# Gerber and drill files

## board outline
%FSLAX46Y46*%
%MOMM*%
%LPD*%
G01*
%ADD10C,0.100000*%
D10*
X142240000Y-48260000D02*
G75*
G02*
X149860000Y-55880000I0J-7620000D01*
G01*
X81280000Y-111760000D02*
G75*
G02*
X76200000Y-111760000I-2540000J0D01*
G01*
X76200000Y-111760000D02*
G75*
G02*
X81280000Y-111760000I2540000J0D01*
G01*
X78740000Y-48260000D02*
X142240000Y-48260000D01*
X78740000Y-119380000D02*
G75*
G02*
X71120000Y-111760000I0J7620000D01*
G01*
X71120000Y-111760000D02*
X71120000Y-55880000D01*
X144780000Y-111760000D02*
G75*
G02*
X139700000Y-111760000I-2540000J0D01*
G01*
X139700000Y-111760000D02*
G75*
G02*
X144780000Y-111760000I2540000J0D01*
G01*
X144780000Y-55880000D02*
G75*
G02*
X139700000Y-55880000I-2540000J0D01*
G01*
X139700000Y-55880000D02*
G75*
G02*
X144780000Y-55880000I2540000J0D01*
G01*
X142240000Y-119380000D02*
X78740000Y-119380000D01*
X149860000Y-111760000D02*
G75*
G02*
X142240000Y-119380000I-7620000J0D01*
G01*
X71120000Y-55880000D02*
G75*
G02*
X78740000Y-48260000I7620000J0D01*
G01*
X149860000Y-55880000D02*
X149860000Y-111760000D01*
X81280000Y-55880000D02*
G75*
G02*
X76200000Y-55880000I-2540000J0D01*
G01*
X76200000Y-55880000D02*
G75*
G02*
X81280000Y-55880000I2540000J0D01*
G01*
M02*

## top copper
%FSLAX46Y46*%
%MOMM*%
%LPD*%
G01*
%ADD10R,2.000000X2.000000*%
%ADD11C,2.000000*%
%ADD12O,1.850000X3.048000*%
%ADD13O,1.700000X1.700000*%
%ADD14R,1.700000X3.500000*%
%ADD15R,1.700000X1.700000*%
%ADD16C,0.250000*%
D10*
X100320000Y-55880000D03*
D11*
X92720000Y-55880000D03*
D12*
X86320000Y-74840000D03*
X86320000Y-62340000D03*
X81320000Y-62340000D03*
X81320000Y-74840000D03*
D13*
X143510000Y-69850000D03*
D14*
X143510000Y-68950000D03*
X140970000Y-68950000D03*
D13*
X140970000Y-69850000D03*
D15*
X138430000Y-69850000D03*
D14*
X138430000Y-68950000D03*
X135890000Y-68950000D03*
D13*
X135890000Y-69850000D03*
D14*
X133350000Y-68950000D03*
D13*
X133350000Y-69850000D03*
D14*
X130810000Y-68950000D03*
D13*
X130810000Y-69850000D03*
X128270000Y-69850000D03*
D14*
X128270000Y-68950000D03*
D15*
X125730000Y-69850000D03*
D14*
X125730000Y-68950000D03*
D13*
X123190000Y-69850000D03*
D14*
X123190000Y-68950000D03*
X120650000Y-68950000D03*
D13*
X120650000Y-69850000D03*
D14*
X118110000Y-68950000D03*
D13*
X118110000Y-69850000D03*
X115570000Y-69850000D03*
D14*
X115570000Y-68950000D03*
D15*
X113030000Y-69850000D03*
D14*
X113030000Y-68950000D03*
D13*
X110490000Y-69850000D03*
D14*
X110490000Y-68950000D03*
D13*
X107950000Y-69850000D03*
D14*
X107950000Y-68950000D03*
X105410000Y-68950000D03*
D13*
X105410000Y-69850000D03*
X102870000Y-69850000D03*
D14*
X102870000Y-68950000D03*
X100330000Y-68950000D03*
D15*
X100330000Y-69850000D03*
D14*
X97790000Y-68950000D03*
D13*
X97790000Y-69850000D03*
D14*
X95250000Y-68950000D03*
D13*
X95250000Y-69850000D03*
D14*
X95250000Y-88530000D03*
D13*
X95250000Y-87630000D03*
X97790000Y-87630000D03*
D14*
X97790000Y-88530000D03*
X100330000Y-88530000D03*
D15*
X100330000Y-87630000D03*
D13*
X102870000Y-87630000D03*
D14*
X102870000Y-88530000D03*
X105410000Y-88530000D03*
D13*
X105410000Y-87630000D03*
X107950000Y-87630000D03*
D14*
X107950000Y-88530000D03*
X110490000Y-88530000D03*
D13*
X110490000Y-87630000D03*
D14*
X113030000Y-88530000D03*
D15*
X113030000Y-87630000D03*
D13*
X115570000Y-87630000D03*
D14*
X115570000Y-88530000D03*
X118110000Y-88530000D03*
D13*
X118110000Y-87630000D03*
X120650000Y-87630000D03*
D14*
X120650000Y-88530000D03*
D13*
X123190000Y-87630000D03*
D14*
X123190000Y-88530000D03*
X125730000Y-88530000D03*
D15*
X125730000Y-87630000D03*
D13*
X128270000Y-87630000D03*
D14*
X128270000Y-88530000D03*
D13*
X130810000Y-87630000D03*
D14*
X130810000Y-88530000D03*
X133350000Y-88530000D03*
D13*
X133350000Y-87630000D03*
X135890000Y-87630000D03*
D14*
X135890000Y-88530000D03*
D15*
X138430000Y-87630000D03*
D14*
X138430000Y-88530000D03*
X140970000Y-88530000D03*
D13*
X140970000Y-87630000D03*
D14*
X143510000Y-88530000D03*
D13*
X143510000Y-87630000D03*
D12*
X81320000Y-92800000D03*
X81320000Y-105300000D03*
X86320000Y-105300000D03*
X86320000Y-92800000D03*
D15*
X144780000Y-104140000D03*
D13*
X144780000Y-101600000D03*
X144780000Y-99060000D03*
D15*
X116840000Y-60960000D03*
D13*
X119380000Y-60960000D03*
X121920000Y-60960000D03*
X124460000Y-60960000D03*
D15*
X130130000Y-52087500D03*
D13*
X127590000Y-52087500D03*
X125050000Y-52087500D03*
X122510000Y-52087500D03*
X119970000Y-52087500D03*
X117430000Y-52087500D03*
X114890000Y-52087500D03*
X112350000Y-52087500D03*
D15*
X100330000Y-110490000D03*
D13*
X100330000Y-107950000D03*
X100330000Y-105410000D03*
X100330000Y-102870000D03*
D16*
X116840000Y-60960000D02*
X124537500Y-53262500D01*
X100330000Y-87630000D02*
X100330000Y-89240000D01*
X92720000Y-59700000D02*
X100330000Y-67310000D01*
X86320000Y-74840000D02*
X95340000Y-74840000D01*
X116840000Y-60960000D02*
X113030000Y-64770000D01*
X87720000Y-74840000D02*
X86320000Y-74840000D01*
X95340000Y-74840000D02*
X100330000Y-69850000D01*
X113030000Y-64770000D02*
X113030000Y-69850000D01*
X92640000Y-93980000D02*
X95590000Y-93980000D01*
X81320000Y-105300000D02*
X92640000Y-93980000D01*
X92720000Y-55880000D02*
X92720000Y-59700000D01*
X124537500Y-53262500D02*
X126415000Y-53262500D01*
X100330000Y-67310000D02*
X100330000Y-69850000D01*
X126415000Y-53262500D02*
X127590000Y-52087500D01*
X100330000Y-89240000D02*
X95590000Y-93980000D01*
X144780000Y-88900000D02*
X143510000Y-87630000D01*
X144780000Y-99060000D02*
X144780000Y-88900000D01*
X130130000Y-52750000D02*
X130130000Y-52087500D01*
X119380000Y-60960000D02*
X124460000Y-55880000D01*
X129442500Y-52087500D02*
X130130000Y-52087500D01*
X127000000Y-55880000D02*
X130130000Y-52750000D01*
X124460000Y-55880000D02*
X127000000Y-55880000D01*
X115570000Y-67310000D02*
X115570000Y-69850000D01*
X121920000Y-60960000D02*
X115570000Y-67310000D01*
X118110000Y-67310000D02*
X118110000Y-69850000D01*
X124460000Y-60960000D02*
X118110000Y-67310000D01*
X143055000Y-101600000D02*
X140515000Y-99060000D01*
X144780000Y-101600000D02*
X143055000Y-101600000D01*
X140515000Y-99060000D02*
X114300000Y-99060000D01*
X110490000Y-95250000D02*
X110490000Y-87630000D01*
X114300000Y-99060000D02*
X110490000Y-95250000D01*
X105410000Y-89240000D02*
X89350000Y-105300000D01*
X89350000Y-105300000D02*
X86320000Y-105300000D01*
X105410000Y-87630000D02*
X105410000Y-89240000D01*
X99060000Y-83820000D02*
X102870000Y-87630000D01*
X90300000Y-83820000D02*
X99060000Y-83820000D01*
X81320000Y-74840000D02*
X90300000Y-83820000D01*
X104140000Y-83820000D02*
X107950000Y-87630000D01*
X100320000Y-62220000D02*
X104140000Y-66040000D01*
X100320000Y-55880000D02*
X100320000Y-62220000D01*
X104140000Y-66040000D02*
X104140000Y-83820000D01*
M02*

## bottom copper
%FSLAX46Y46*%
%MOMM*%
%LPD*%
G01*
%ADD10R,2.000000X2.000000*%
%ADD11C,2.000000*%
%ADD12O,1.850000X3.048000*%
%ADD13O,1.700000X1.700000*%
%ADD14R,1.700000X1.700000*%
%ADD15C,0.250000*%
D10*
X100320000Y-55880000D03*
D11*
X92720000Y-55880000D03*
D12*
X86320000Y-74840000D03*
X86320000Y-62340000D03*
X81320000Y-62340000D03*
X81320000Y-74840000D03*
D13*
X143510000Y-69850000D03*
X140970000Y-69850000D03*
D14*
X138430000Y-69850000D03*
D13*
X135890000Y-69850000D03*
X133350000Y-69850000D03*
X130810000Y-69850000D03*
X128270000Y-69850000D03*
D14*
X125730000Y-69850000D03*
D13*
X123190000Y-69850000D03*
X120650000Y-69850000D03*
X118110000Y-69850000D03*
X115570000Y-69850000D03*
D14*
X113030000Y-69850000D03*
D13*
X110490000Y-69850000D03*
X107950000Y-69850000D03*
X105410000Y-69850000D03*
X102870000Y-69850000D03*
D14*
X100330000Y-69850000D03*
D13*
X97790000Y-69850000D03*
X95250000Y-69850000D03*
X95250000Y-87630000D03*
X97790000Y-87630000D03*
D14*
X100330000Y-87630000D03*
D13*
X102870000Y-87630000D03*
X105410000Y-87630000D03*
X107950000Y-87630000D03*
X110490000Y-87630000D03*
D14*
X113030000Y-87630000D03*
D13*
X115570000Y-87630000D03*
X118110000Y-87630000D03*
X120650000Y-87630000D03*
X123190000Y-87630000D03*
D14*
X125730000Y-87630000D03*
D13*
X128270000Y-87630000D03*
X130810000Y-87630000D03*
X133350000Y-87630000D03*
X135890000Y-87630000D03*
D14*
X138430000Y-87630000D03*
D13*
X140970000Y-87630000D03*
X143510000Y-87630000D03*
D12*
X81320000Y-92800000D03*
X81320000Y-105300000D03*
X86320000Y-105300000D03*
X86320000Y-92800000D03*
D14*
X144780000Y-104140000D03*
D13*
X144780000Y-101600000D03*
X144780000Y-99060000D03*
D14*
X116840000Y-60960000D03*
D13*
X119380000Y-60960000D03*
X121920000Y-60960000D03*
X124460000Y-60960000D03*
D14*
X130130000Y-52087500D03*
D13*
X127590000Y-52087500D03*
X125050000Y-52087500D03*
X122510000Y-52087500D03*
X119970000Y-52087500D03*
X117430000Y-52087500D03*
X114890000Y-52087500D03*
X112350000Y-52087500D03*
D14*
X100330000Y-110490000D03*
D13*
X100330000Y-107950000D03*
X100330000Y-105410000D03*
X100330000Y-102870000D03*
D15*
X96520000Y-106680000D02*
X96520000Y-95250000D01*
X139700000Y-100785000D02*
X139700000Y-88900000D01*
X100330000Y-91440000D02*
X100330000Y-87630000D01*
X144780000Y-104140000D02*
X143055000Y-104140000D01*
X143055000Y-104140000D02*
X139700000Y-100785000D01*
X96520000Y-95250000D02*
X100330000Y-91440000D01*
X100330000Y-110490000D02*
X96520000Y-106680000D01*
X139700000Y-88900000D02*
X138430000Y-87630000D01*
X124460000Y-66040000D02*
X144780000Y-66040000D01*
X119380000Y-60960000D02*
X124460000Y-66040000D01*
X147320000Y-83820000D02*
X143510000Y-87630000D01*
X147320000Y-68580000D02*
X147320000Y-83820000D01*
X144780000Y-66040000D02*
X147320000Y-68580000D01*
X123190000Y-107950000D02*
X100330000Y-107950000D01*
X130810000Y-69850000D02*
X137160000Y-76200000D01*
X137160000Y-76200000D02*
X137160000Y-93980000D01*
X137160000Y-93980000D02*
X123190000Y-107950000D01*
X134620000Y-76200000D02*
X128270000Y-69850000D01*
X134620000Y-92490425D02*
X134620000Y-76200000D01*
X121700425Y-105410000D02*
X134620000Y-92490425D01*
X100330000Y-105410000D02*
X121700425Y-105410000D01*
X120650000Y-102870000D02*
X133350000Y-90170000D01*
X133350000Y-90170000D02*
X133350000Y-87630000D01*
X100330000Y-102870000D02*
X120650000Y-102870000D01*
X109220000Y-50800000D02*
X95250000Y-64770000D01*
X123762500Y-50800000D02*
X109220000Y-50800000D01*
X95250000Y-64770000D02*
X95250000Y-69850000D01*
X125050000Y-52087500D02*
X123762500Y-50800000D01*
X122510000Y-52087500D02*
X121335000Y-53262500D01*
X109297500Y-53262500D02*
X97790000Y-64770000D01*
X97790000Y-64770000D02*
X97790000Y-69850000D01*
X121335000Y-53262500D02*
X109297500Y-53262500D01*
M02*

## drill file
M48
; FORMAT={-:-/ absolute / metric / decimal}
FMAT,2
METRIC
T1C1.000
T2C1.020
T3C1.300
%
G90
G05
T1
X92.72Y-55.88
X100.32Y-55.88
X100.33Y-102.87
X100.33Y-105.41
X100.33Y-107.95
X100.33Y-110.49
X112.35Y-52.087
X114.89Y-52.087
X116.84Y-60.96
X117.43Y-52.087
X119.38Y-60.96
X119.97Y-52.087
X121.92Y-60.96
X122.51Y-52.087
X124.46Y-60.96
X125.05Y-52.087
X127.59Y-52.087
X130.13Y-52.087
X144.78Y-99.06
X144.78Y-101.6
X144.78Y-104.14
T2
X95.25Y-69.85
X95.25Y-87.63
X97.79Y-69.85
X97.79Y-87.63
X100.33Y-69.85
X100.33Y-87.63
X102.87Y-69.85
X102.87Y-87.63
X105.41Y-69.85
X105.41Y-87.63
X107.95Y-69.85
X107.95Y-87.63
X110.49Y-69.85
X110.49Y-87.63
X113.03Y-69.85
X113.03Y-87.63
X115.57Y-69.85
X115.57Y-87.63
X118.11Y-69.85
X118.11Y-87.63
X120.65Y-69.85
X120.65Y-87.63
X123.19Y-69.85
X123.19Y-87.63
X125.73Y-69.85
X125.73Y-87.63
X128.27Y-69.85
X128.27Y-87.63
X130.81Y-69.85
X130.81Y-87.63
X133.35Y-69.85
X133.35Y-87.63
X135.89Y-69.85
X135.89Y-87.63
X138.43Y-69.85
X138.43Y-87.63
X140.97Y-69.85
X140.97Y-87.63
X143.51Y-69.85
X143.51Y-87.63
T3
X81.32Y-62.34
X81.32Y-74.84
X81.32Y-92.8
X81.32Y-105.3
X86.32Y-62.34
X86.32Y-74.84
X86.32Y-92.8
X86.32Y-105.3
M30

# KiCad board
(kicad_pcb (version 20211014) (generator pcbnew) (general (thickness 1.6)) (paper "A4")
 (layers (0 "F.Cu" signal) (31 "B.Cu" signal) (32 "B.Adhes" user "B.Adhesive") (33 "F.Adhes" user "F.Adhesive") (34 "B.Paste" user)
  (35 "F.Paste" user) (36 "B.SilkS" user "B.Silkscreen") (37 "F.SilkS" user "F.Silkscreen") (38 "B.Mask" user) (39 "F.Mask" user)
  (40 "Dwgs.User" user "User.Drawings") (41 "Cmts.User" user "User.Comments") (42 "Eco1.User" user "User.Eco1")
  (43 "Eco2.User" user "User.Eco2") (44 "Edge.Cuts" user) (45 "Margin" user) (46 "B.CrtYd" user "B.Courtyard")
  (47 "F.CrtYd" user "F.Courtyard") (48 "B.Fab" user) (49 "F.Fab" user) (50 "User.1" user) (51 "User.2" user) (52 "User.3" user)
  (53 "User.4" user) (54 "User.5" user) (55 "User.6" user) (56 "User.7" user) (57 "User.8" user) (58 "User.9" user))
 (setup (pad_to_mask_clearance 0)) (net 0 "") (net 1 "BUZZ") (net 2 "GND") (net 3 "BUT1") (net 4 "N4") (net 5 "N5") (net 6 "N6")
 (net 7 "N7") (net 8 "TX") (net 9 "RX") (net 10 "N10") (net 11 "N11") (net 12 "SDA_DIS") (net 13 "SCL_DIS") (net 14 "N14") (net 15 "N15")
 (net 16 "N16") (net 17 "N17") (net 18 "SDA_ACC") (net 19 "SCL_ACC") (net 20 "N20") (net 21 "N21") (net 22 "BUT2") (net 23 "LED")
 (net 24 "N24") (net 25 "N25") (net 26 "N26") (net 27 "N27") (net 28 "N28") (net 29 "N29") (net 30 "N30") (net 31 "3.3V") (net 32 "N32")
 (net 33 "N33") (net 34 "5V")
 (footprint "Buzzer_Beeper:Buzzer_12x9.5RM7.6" (layer "F.Cu") (at 100.32 55.88 180)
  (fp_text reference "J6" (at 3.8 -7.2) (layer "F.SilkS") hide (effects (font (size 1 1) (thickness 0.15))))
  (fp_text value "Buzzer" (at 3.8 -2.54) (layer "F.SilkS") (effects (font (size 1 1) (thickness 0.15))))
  (pad "1" thru_hole rect (at 0 0 180) (size 2 2) (drill 1) (layers *.Cu *.Mask) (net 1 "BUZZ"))
  (pad "2" thru_hole circle (at 7.6 0 180) (size 2 2) (drill 1) (layers *.Cu *.Mask) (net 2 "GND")))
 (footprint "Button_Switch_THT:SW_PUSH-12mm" (layer "F.Cu") (at 86.32 62.34 -90)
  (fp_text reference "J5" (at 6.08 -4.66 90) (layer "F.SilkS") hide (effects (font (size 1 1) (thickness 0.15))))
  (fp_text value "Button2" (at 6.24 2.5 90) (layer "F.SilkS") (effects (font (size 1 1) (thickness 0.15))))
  (pad "1" thru_hole oval (at 12.5 0 270) (size 3.048 1.85) (drill 1.3) (layers *.Cu *.Mask) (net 2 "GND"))
  (pad "1" thru_hole oval (at 0 0 270) (size 3.048 1.85) (drill 1.3) (layers *.Cu *.Mask) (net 2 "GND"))
  (pad "2" thru_hole oval (at 0 5 270) (size 3.048 1.85) (drill 1.3) (layers *.Cu *.Mask) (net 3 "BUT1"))
  (pad "2" thru_hole oval (at 12.5 5 270) (size 3.048 1.85) (drill 1.3) (layers *.Cu *.Mask) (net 3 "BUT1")))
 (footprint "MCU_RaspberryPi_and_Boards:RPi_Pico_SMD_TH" (layer "F.Cu") (at 119.38 78.74 -90)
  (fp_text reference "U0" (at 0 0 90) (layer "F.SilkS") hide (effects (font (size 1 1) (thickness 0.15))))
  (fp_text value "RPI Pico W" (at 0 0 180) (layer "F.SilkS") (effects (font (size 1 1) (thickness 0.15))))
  (pad "1" thru_hole oval (at -8.89 -24.13 270) (size 1.7 1.7) (drill 1.02) (layers *.Cu *.Mask) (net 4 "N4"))
  (pad "1" smd rect (at -8.89 -24.13 270) (size 3.5 1.7) (drill (offset -0.9 0)) (layers "F.Cu" "F.Mask") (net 4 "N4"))
  (pad "2" smd rect (at -8.89 -21.59 270) (size 3.5 1.7) (drill (offset -0.9 0)) (layers "F.Cu" "F.Mask") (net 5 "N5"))
  (pad "2" thru_hole oval (at -8.89 -21.59 270) (size 1.7 1.7) (drill 1.02) (layers *.Cu *.Mask) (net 5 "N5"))
  (pad "3" thru_hole rect (at -8.89 -19.05 270) (size 1.7 1.7) (drill 1.02) (layers *.Cu *.Mask) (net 2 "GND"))
  (pad "3" smd rect (at -8.89 -19.05 270) (size 3.5 1.7) (drill (offset -0.9 0)) (layers "F.Cu" "F.Mask") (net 2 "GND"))
  (pad "4" smd rect (at -8.89 -16.51 270) (size 3.5 1.7) (drill (offset -0.9 0)) (layers "F.Cu" "F.Mask") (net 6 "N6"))
  (pad "4" thru_hole oval (at -8.89 -16.51 270) (size 1.7 1.7) (drill 1.02) (layers *.Cu *.Mask) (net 6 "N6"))
  (pad "5" smd rect (at -8.89 -13.97 270) (size 3.5 1.7) (drill (offset -0.9 0)) (layers "F.Cu" "F.Mask") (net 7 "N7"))
  (pad "5" thru_hole oval (at -8.89 -13.97 270) (size 1.7 1.7) (drill 1.02) (layers *.Cu *.Mask) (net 7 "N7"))
  (pad "6" smd rect (at -8.89 -11.43 270) (size 3.5 1.7) (drill (offset -0.9 0)) (layers "F.Cu" "F.Mask") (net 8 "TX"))
  (pad "6" thru_hole oval (at -8.89 -11.43 270) (size 1.7 1.7) (drill 1.02) (layers *.Cu *.Mask) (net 8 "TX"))
  (pad "7" thru_hole oval (at -8.89 -8.89 270) (size 1.7 1.7) (drill 1.02) (layers *.Cu *.Mask) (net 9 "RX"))
  (pad "7" smd rect (at -8.89 -8.89 270) (size 3.5 1.7) (drill (offset -0.9 0)) (layers "F.Cu" "F.Mask") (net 9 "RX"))
  (pad "8" thru_hole rect (at -8.89 -6.35 270) (size 1.7 1.7) (drill 1.02) (layers *.Cu *.Mask) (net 2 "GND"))
  (pad "8" smd rect (at -8.89 -6.35 270) (size 3.5 1.7) (drill (offset -0.9 0)) (layers "F.Cu" "F.Mask") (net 2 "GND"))
  (pad "9" thru_hole oval (at -8.89 -3.81 270) (size 1.7 1.7) (drill 1.02) (layers *.Cu *.Mask) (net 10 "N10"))
  (pad "9" smd rect (at -8.89 -3.81 270) (size 3.5 1.7) (drill (offset -0.9 0)) (layers "F.Cu" "F.Mask") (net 10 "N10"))
  (pad "10" smd rect (at -8.89 -1.27 270) (size 3.5 1.7) (drill (offset -0.9 0)) (layers "F.Cu" "F.Mask") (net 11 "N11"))
  (pad "10" thru_hole oval (at -8.89 -1.27 270) (size 1.7 1.7) (drill 1.02) (layers *.Cu *.Mask) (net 11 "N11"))
  (pad "11" smd rect (at -8.89 1.27 270) (size 3.5 1.7) (drill (offset -0.9 0)) (layers "F.Cu" "F.Mask") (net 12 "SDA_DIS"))
  (pad "11" thru_hole oval (at -8.89 1.27 270) (size 1.7 1.7) (drill 1.02) (layers *.Cu *.Mask) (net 12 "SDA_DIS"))
  (pad "12" thru_hole oval (at -8.89 3.81 270) (size 1.7 1.7) (drill 1.02) (layers *.Cu *.Mask) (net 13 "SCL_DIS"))
  (pad "12" smd rect (at -8.89 3.81 270) (size 3.5 1.7) (drill (offset -0.9 0)) (layers "F.Cu" "F.Mask") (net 13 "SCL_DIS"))
  (pad "13" thru_hole rect (at -8.89 6.35 270) (size 1.7 1.7) (drill 1.02) (layers *.Cu *.Mask) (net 2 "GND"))
  (pad "13" smd rect (at -8.89 6.35 270) (size 3.5 1.7) (drill (offset -0.9 0)) (layers "F.Cu" "F.Mask") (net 2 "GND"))
  (pad "14" thru_hole oval (at -8.89 8.89 270) (size 1.7 1.7) (drill 1.02) (layers *.Cu *.Mask) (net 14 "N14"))
  (pad "14" smd rect (at -8.89 8.89 270) (size 3.5 1.7) (drill (offset -0.9 0)) (layers "F.Cu" "F.Mask") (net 14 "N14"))
  (pad "15" thru_hole oval (at -8.89 11.43 270) (size 1.7 1.7) (drill 1.02) (layers *.Cu *.Mask) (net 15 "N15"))
  (pad "15" smd rect (at -8.89 11.43 270) (size 3.5 1.7) (drill (offset -0.9 0)) (layers "F.Cu" "F.Mask") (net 15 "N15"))
  (pad "16" smd rect (at -8.89 13.97 270) (size 3.5 1.7) (drill (offset -0.9 0)) (layers "F.Cu" "F.Mask") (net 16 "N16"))
  (pad "16" thru_hole oval (at -8.89 13.97 270) (size 1.7 1.7) (drill 1.02) (layers *.Cu *.Mask) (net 16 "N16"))
  (pad "17" thru_hole oval (at -8.89 16.51 270) (size 1.7 1.7) (drill 1.02) (layers *.Cu *.Mask) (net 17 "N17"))
  (pad "17" smd rect (at -8.89 16.51 270) (size 3.5 1.7) (drill (offset -0.9 0)) (layers "F.Cu" "F.Mask") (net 17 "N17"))
  (pad "18" smd rect (at -8.89 19.05 270) (size 3.5 1.7) (drill (offset -0.9 0)) (layers "F.Cu" "F.Mask") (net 2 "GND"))
  (pad "18" thru_hole rect (at -8.89 19.05 270) (size 1.7 1.7) (drill 1.02) (layers *.Cu *.Mask) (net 2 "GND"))
  (pad "19" smd rect (at -8.89 21.59 270) (size 3.5 1.7) (drill (offset -0.9 0)) (layers "F.Cu" "F.Mask") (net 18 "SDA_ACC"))
  (pad "19" thru_hole oval (at -8.89 21.59 270) (size 1.7 1.7) (drill 1.02) (layers *.Cu *.Mask) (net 18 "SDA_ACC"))
  (pad "20" smd rect (at -8.89 24.13 270) (size 3.5 1.7) (drill (offset -0.9 0)) (layers "F.Cu" "F.Mask") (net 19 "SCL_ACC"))
  (pad "20" thru_hole oval (at -8.89 24.13 270) (size 1.7 1.7) (drill 1.02) (layers *.Cu *.Mask) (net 19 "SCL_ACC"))
  (pad "21" smd rect (at 8.89 24.13 270) (size 3.5 1.7) (drill (offset 0.9 0)) (layers "F.Cu" "F.Mask") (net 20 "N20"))
  (pad "21" thru_hole oval (at 8.89 24.13 270) (size 1.7 1.7) (drill 1.02) (layers *.Cu *.Mask) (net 20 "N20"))
  (pad "22" thru_hole oval (at 8.89 21.59 270) (size 1.7 1.7) (drill 1.02) (layers *.Cu *.Mask) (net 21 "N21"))
  (pad "22" smd rect (at 8.89 21.59 270) (size 3.5 1.7) (drill (offset 0.9 0)) (layers "F.Cu" "F.Mask") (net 21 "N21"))
  (pad "23" smd rect (at 8.89 19.05 270) (size 3.5 1.7) (drill (offset 0.9 0)) (layers "F.Cu" "F.Mask") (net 2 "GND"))
  (pad "23" thru_hole rect (at 8.89 19.05 270) (size 1.7 1.7) (drill 1.02) (layers *.Cu *.Mask) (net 2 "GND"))
  (pad "24" thru_hole oval (at 8.89 16.51 270) (size 1.7 1.7) (drill 1.02) (layers *.Cu *.Mask) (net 3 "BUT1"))
  (pad "24" smd rect (at 8.89 16.51 270) (size 3.5 1.7) (drill (offset 0.9 0)) (layers "F.Cu" "F.Mask") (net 3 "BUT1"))
  (pad "25" smd rect (at 8.89 13.97 270) (size 3.5 1.7) (drill (offset 0.9 0)) (layers "F.Cu" "F.Mask") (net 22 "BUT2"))
  (pad "25" thru_hole oval (at 8.89 13.97 270) (size 1.7 1.7) (drill 1.02) (layers *.Cu *.Mask) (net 22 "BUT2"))
  (pad "26" thru_hole oval (at 8.89 11.43 270) (size 1.7 1.7) (drill 1.02) (layers *.Cu *.Mask) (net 1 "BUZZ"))
  (pad "26" smd rect (at 8.89 11.43 270) (size 3.5 1.7) (drill (offset 0.9 0)) (layers "F.Cu" "F.Mask") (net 1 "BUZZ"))
  (pad "27" smd rect (at 8.89 8.89 270) (size 3.5 1.7) (drill (offset 0.9 0)) (layers "F.Cu" "F.Mask") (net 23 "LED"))
  (pad "27" thru_hole oval (at 8.89 8.89 270) (size 1.7 1.7) (drill 1.02) (layers *.Cu *.Mask) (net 23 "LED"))
  (pad "28" smd rect (at 8.89 6.35 270) (size 3.5 1.7) (drill (offset 0.9 0)) (layers "F.Cu" "F.Mask") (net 2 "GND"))
  (pad "28" thru_hole rect (at 8.89 6.35 270) (size 1.7 1.7) (drill 1.02) (layers *.Cu *.Mask) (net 2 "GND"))
  (pad "29" thru_hole oval (at 8.89 3.81 270) (size 1.7 1.7) (drill 1.02) (layers *.Cu *.Mask) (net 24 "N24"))
  (pad "29" smd rect (at 8.89 3.81 270) (size 3.5 1.7) (drill (offset 0.9 0)) (layers "F.Cu" "F.Mask") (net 24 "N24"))
  (pad "30" smd rect (at 8.89 1.27 270) (size 3.5 1.7) (drill (offset 0.9 0)) (layers "F.Cu" "F.Mask") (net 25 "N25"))
  (pad "30" thru_hole oval (at 8.89 1.27 270) (size 1.7 1.7) (drill 1.02) (layers *.Cu *.Mask) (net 25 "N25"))
  (pad "31" thru_hole oval (at 8.89 -1.27 270) (size 1.7 1.7) (drill 1.02) (layers *.Cu *.Mask) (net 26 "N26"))
  (pad "31" smd rect (at 8.89 -1.27 270) (size 3.5 1.7) (drill (offset 0.9 0)) (layers "F.Cu" "F.Mask") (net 26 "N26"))
  (pad "32" thru_hole oval (at 8.89 -3.81 270) (size 1.7 1.7) (drill 1.02) (layers *.Cu *.Mask) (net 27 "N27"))
  (pad "32" smd rect (at 8.89 -3.81 270) (size 3.5 1.7) (drill (offset 0.9 0)) (layers "F.Cu" "F.Mask") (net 27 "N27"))
  (pad "33" smd rect (at 8.89 -6.35 270) (size 3.5 1.7) (drill (offset 0.9 0)) (layers "F.Cu" "F.Mask") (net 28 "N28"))
  (pad "33" thru_hole rect (at 8.89 -6.35 270) (size 1.7 1.7) (drill 1.02) (layers *.Cu *.Mask) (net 28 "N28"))
  (pad "34" thru_hole oval (at 8.89 -8.89 270) (size 1.7 1.7) (drill 1.02) (layers *.Cu *.Mask) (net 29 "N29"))
  (pad "34" smd rect (at 8.89 -8.89 270) (size 3.5 1.7) (drill (offset 0.9 0)) (layers "F.Cu" "F.Mask") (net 29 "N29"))
  (pad "35" thru_hole oval (at 8.89 -11.43 270) (size 1.7 1.7) (drill 1.02) (layers *.Cu *.Mask) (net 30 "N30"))
  (pad "35" smd rect (at 8.89 -11.43 270) (size 3.5 1.7) (drill (offset 0.9 0)) (layers "F.Cu" "F.Mask") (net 30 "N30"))
  (pad "36" smd rect (at 8.89 -13.97 270) (size 3.5 1.7) (drill (offset 0.9 0)) (layers "F.Cu" "F.Mask") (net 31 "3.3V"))
  (pad "36" thru_hole oval (at 8.89 -13.97 270) (size 1.7 1.7) (drill 1.02) (layers *.Cu *.Mask) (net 31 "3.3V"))
  (pad "37" thru_hole oval (at 8.89 -16.51 270) (size 1.7 1.7) (drill 1.02) (layers *.Cu *.Mask) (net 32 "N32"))
  (pad "37" smd rect (at 8.89 -16.51 270) (size 3.5 1.7) (drill (offset 0.9 0)) (layers "F.Cu" "F.Mask") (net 32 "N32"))
  (pad "38" thru_hole rect (at 8.89 -19.05 270) (size 1.7 1.7) (drill 1.02) (layers *.Cu *.Mask) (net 2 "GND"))
  (pad "38" smd rect (at 8.89 -19.05 270) (size 3.5 1.7) (drill (offset 0.9 0)) (layers "F.Cu" "F.Mask") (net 2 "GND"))
  (pad "39" smd rect (at 8.89 -21.59 270) (size 3.5 1.7) (drill (offset 0.9 0)) (layers "F.Cu" "F.Mask") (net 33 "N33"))
  (pad "39" thru_hole oval (at 8.89 -21.59 270) (size 1.7 1.7) (drill 1.02) (layers *.Cu *.Mask) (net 33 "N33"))
  (pad "40" smd rect (at 8.89 -24.13 270) (size 3.5 1.7) (drill (offset 0.9 0)) (layers "F.Cu" "F.Mask") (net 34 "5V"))
  (pad "40" thru_hole oval (at 8.89 -24.13 270) (size 1.7 1.7) (drill 1.02) (layers *.Cu *.Mask) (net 34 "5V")))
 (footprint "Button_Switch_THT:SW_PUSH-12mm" (layer "F.Cu") (at 81.32 105.3 90)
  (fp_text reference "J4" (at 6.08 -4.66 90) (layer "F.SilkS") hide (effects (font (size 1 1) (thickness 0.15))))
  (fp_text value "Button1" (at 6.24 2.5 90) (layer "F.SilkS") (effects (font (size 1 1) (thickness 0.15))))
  (pad "1" thru_hole oval (at 12.5 0 90) (size 3.048 1.85) (drill 1.3) (layers *.Cu *.Mask) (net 2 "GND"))
  (pad "1" thru_hole oval (at 0 0 90) (size 3.048 1.85) (drill 1.3) (layers *.Cu *.Mask) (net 2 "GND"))
  (pad "2" thru_hole oval (at 0 5 90) (size 3.048 1.85) (drill 1.3) (layers *.Cu *.Mask) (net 22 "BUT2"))
  (pad "2" thru_hole oval (at 12.5 5 90) (size 3.048 1.85) (drill 1.3) (layers *.Cu *.Mask) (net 22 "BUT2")))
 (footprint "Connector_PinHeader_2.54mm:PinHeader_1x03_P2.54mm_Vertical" (layer "F.Cu") (at 144.78 104.14 180)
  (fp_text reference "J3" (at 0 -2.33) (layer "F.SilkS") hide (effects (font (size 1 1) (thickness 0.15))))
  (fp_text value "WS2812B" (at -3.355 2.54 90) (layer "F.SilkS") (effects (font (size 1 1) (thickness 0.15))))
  (pad "1" thru_hole rect (at 0 0 180) (size 1.7 1.7) (drill 1) (layers *.Cu *.Mask) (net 2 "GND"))
  (pad "2" thru_hole oval (at 0 2.54 180) (size 1.7 1.7) (drill 1) (layers *.Cu *.Mask) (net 23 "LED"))
  (pad "3" thru_hole oval (at 0 5.08 180) (size 1.7 1.7) (drill 1) (layers *.Cu *.Mask) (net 34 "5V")))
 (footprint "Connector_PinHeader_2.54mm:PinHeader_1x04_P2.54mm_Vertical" (layer "F.Cu") (at 116.84 60.96 90)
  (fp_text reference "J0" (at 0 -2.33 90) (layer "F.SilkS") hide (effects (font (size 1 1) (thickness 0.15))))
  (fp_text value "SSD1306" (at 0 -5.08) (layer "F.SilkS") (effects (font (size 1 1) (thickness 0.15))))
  (pad "1" thru_hole rect (at 0 0 90) (size 1.7 1.7) (drill 1) (layers *.Cu *.Mask) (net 2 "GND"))
  (pad "2" thru_hole oval (at 0 2.54 90) (size 1.7 1.7) (drill 1) (layers *.Cu *.Mask) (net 34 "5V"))
  (pad "3" thru_hole oval (at 0 5.08 90) (size 1.7 1.7) (drill 1) (layers *.Cu *.Mask) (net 13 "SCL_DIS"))
  (pad "4" thru_hole oval (at 0 7.62 90) (size 1.7 1.7) (drill 1) (layers *.Cu *.Mask) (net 12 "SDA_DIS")))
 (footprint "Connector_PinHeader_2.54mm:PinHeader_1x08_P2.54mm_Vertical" (layer "F.Cu") (at 130.13 52.0875 -90)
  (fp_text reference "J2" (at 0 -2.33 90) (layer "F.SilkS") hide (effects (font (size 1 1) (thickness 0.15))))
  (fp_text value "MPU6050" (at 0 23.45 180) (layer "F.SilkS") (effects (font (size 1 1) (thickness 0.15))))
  (pad "1" thru_hole rect (at 0 0 270) (size 1.7 1.7) (drill 1) (layers *.Cu *.Mask) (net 34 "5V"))
  (pad "2" thru_hole oval (at 0 2.54 270) (size 1.7 1.7) (drill 1) (layers *.Cu *.Mask) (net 2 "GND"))
  (pad "3" thru_hole oval (at 0 5.08 270) (size 1.7 1.7) (drill 1) (layers *.Cu *.Mask) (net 19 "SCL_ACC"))
  (pad "4" thru_hole oval (at 0 7.62 270) (size 1.7 1.7) (drill 1) (layers *.Cu *.Mask) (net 18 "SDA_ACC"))
  (pad "5" thru_hole oval (at 0 10.16 270) (size 1.7 1.7) (drill 1) (layers *.Cu *.Mask))
  (pad "6" thru_hole oval (at 0 12.7 270) (size 1.7 1.7) (drill 1) (layers *.Cu *.Mask))
  (pad "7" thru_hole oval (at 0 15.24 270) (size 1.7 1.7) (drill 1) (layers *.Cu *.Mask))
  (pad "8" thru_hole oval (at 0 17.78 270) (size 1.7 1.7) (drill 1) (layers *.Cu *.Mask)))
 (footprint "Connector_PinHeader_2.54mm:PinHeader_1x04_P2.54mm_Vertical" (layer "F.Cu") (at 100.33 110.49 180)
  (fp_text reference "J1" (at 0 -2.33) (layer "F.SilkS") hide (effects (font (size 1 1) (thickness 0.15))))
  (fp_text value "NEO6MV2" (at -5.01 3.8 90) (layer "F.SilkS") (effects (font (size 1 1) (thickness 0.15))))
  (pad "1" thru_hole rect (at 0 0 180) (size 1.7 1.7) (drill 1) (layers *.Cu *.Mask) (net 2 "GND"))
  (pad "2" thru_hole oval (at 0 2.54 180) (size 1.7 1.7) (drill 1) (layers *.Cu *.Mask) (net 8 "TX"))
  (pad "3" thru_hole oval (at 0 5.08 180) (size 1.7 1.7) (drill 1) (layers *.Cu *.Mask) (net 9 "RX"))
  (pad "4" thru_hole oval (at 0 7.62 180) (size 1.7 1.7) (drill 1) (layers *.Cu *.Mask) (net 31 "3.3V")))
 (gr_arc (start 142.24 48.26) (mid 147.628154 50.491846) (end 149.86 55.88) (layer "Edge.Cuts") (width 0.1))
 (gr_circle (center 78.74 111.76) (end 81.28 111.76) (layer "Edge.Cuts") (width 0.1) (fill none))
 (gr_line (start 78.74 48.26) (end 142.24 48.26) (layer "Edge.Cuts") (width 0.1))
 (gr_arc (start 78.74 119.38) (mid 73.351846 117.148154) (end 71.12 111.76) (layer "Edge.Cuts") (width 0.1))
 (gr_line (start 71.12 111.76) (end 71.12 55.88) (layer "Edge.Cuts") (width 0.1))
 (gr_circle (center 142.24 111.76) (end 144.78 111.76) (layer "Edge.Cuts") (width 0.1) (fill none))
 (gr_circle (center 142.24 55.88) (end 144.78 55.88) (layer "Edge.Cuts") (width 0.1) (fill none))
 (gr_line (start 142.24 119.38) (end 78.74 119.38) (layer "Edge.Cuts") (width 0.1))
 (gr_arc (start 149.86 111.76) (mid 147.628154 117.148154) (end 142.24 119.38) (layer "Edge.Cuts") (width 0.1))
 (gr_arc (start 71.12 55.88) (mid 73.351846 50.491846) (end 78.74 48.26) (layer "Edge.Cuts") (width 0.1))
 (gr_line (start 149.86 55.88) (end 149.86 111.76) (layer "Edge.Cuts") (width 0.1))
 (gr_circle (center 78.74 55.88) (end 81.28 55.88) (layer "Edge.Cuts") (width 0.1) (fill none))
 (segment (start 116.84 60.96) (end 124.5375 53.2625) (width 0.25) (layer "F.Cu") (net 2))
 (segment (start 100.33 87.63) (end 100.33 89.24) (width 0.25) (layer "F.Cu") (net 2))
 (segment (start 92.72 59.7) (end 100.33 67.31) (width 0.25) (layer "F.Cu") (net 2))
 (segment (start 86.32 74.84) (end 95.34 74.84) (width 0.25) (layer "F.Cu") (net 2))
 (segment (start 116.84 60.96) (end 113.03 64.77) (width 0.25) (layer "F.Cu") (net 2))
 (segment (start 87.72 74.84) (end 86.32 74.84) (width 0.25) (layer "F.Cu") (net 2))
 (segment (start 95.34 74.84) (end 100.33 69.85) (width 0.25) (layer "F.Cu") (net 2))
 (segment (start 113.03 64.77) (end 113.03 69.85) (width 0.25) (layer "F.Cu") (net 2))
 (segment (start 92.64 93.98) (end 95.59 93.98) (width 0.25) (layer "F.Cu") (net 2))
 (segment (start 81.32 105.3) (end 92.64 93.98) (width 0.25) (layer "F.Cu") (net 2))
 (segment (start 92.72 55.88) (end 92.72 59.7) (width 0.25) (layer "F.Cu") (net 2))
 (segment (start 124.5375 53.2625) (end 126.415 53.2625) (width 0.25) (layer "F.Cu") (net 2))
 (segment (start 100.33 67.31) (end 100.33 69.85) (width 0.25) (layer "F.Cu") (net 2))
 (segment (start 126.415 53.2625) (end 127.59 52.0875) (width 0.25) (layer "F.Cu") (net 2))
 (segment (start 100.33 89.24) (end 95.59 93.98) (width 0.25) (layer "F.Cu") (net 2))
 (segment (start 96.52 106.68) (end 96.52 95.25) (width 0.25) (layer "B.Cu") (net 2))
 (segment (start 139.7 100.785) (end 139.7 88.9) (width 0.25) (layer "B.Cu") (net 2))
 (segment (start 100.33 91.44) (end 100.33 87.63) (width 0.25) (layer "B.Cu") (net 2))
 (segment (start 144.78 104.14) (end 143.055 104.14) (width 0.25) (layer "B.Cu") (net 2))
 (segment (start 143.055 104.14) (end 139.7 100.785) (width 0.25) (layer "B.Cu") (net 2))
 (segment (start 96.52 95.25) (end 100.33 91.44) (width 0.25) (layer "B.Cu") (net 2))
 (segment (start 100.33 110.49) (end 96.52 106.68) (width 0.25) (layer "B.Cu") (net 2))
 (segment (start 139.7 88.9) (end 138.43 87.63) (width 0.25) (layer "B.Cu") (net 2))
 (segment (start 144.78 88.9) (end 143.51 87.63) (width 0.25) (layer "F.Cu") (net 34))
 (segment (start 144.78 99.06) (end 144.78 88.9) (width 0.25) (layer "F.Cu") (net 34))
 (segment (start 130.13 52.75) (end 130.13 52.0875) (width 0.25) (layer "F.Cu") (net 34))
 (segment (start 119.38 60.96) (end 124.46 55.88) (width 0.25) (layer "F.Cu") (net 34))
 (segment (start 129.4425 52.0875) (end 130.13 52.0875) (width 0.25) (layer "F.Cu") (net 34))
 (segment (start 127 55.88) (end 130.13 52.75) (width 0.25) (layer "F.Cu") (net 34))
 (segment (start 124.46 55.88) (end 127 55.88) (width 0.25) (layer "F.Cu") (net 34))
 (segment (start 124.46 66.04) (end 144.78 66.04) (width 0.25) (layer "B.Cu") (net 34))
 (segment (start 119.38 60.96) (end 124.46 66.04) (width 0.25) (layer "B.Cu") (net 34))
 (segment (start 147.32 83.82) (end 143.51 87.63) (width 0.25) (layer "B.Cu") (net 34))
 (segment (start 147.32 68.58) (end 147.32 83.82) (width 0.25) (layer "B.Cu") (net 34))
 (segment (start 144.78 66.04) (end 147.32 68.58) (width 0.25) (layer "B.Cu") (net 34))
 (segment (start 115.57 67.31) (end 115.57 69.85) (width 0.25) (layer "F.Cu") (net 13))
 (segment (start 121.92 60.96) (end 115.57 67.31) (width 0.25) (layer "F.Cu") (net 13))
 (segment (start 118.11 67.31) (end 118.11 69.85) (width 0.25) (layer "F.Cu") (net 12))
 (segment (start 124.46 60.96) (end 118.11 67.31) (width 0.25) (layer "F.Cu") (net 12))
 (segment (start 123.19 107.95) (end 100.33 107.95) (width 0.25) (layer "B.Cu") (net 8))
 (segment (start 130.81 69.85) (end 137.16 76.2) (width 0.25) (layer "B.Cu") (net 8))
 (segment (start 137.16 76.2) (end 137.16 93.98) (width 0.25) (layer "B.Cu") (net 8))
 (segment (start 137.16 93.98) (end 123.19 107.95) (width 0.25) (layer "B.Cu") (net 8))
 (segment (start 134.62 76.2) (end 128.27 69.85) (width 0.25) (layer "B.Cu") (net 9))
 (segment (start 134.62 92.490425) (end 134.62 76.2) (width 0.25) (layer "B.Cu") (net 9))
 (segment (start 121.700425 105.41) (end 134.62 92.490425) (width 0.25) (layer "B.Cu") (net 9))
 (segment (start 100.33 105.41) (end 121.700425 105.41) (width 0.25) (layer "B.Cu") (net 9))
 (segment (start 120.65 102.87) (end 133.35 90.17) (width 0.25) (layer "B.Cu") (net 31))
 (segment (start 133.35 90.17) (end 133.35 87.63) (width 0.25) (layer "B.Cu") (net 31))
 (segment (start 100.33 102.87) (end 120.65 102.87) (width 0.25) (layer "B.Cu") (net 31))
 (segment (start 109.22 50.8) (end 95.25 64.77) (width 0.25) (layer "B.Cu") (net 19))
 (segment (start 123.7625 50.8) (end 109.22 50.8) (width 0.25) (layer "B.Cu") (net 19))
 (segment (start 95.25 64.77) (end 95.25 69.85) (width 0.25) (layer "B.Cu") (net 19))
 (segment (start 125.05 52.0875) (end 123.7625 50.8) (width 0.25) (layer "B.Cu") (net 19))
 (segment (start 122.51 52.0875) (end 121.335 53.2625) (width 0.25) (layer "B.Cu") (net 18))
 (segment (start 109.2975 53.2625) (end 97.79 64.77) (width 0.25) (layer "B.Cu") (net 18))
 (segment (start 97.79 64.77) (end 97.79 69.85) (width 0.25) (layer "B.Cu") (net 18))
 (segment (start 121.335 53.2625) (end 109.2975 53.2625) (width 0.25) (layer "B.Cu") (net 18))
 (segment (start 143.055 101.6) (end 140.515 99.06) (width 0.25) (layer "F.Cu") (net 23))
 (segment (start 144.78 101.6) (end 143.055 101.6) (width 0.25) (layer "F.Cu") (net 23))
 (segment (start 140.515 99.06) (end 114.3 99.06) (width 0.25) (layer "F.Cu") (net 23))
 (segment (start 110.49 95.25) (end 110.49 87.63) (width 0.25) (layer "F.Cu") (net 23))
 (segment (start 114.3 99.06) (end 110.49 95.25) (width 0.25) (layer "F.Cu") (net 23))
 (segment (start 105.41 89.24) (end 89.35 105.3) (width 0.25) (layer "F.Cu") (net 22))
 (segment (start 89.35 105.3) (end 86.32 105.3) (width 0.25) (layer "F.Cu") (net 22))
 (segment (start 105.41 87.63) (end 105.41 89.24) (width 0.25) (layer "F.Cu") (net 22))
 (segment (start 99.06 83.82) (end 102.87 87.63) (width 0.25) (layer "F.Cu") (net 3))
 (segment (start 90.3 83.82) (end 99.06 83.82) (width 0.25) (layer "F.Cu") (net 3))
 (segment (start 81.32 74.84) (end 90.3 83.82) (width 0.25) (layer "F.Cu") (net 3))
 (segment (start 104.14 83.82) (end 107.95 87.63) (width 0.25) (layer "F.Cu") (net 1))
 (segment (start 100.32 62.22) (end 104.14 66.04) (width 0.25) (layer "F.Cu") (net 1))
 (segment (start 100.32 55.88) (end 100.32 62.22) (width 0.25) (layer "F.Cu") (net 1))
 (segment (start 104.14 66.04) (end 104.14 83.82) (width 0.25) (layer "F.Cu") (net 1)))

